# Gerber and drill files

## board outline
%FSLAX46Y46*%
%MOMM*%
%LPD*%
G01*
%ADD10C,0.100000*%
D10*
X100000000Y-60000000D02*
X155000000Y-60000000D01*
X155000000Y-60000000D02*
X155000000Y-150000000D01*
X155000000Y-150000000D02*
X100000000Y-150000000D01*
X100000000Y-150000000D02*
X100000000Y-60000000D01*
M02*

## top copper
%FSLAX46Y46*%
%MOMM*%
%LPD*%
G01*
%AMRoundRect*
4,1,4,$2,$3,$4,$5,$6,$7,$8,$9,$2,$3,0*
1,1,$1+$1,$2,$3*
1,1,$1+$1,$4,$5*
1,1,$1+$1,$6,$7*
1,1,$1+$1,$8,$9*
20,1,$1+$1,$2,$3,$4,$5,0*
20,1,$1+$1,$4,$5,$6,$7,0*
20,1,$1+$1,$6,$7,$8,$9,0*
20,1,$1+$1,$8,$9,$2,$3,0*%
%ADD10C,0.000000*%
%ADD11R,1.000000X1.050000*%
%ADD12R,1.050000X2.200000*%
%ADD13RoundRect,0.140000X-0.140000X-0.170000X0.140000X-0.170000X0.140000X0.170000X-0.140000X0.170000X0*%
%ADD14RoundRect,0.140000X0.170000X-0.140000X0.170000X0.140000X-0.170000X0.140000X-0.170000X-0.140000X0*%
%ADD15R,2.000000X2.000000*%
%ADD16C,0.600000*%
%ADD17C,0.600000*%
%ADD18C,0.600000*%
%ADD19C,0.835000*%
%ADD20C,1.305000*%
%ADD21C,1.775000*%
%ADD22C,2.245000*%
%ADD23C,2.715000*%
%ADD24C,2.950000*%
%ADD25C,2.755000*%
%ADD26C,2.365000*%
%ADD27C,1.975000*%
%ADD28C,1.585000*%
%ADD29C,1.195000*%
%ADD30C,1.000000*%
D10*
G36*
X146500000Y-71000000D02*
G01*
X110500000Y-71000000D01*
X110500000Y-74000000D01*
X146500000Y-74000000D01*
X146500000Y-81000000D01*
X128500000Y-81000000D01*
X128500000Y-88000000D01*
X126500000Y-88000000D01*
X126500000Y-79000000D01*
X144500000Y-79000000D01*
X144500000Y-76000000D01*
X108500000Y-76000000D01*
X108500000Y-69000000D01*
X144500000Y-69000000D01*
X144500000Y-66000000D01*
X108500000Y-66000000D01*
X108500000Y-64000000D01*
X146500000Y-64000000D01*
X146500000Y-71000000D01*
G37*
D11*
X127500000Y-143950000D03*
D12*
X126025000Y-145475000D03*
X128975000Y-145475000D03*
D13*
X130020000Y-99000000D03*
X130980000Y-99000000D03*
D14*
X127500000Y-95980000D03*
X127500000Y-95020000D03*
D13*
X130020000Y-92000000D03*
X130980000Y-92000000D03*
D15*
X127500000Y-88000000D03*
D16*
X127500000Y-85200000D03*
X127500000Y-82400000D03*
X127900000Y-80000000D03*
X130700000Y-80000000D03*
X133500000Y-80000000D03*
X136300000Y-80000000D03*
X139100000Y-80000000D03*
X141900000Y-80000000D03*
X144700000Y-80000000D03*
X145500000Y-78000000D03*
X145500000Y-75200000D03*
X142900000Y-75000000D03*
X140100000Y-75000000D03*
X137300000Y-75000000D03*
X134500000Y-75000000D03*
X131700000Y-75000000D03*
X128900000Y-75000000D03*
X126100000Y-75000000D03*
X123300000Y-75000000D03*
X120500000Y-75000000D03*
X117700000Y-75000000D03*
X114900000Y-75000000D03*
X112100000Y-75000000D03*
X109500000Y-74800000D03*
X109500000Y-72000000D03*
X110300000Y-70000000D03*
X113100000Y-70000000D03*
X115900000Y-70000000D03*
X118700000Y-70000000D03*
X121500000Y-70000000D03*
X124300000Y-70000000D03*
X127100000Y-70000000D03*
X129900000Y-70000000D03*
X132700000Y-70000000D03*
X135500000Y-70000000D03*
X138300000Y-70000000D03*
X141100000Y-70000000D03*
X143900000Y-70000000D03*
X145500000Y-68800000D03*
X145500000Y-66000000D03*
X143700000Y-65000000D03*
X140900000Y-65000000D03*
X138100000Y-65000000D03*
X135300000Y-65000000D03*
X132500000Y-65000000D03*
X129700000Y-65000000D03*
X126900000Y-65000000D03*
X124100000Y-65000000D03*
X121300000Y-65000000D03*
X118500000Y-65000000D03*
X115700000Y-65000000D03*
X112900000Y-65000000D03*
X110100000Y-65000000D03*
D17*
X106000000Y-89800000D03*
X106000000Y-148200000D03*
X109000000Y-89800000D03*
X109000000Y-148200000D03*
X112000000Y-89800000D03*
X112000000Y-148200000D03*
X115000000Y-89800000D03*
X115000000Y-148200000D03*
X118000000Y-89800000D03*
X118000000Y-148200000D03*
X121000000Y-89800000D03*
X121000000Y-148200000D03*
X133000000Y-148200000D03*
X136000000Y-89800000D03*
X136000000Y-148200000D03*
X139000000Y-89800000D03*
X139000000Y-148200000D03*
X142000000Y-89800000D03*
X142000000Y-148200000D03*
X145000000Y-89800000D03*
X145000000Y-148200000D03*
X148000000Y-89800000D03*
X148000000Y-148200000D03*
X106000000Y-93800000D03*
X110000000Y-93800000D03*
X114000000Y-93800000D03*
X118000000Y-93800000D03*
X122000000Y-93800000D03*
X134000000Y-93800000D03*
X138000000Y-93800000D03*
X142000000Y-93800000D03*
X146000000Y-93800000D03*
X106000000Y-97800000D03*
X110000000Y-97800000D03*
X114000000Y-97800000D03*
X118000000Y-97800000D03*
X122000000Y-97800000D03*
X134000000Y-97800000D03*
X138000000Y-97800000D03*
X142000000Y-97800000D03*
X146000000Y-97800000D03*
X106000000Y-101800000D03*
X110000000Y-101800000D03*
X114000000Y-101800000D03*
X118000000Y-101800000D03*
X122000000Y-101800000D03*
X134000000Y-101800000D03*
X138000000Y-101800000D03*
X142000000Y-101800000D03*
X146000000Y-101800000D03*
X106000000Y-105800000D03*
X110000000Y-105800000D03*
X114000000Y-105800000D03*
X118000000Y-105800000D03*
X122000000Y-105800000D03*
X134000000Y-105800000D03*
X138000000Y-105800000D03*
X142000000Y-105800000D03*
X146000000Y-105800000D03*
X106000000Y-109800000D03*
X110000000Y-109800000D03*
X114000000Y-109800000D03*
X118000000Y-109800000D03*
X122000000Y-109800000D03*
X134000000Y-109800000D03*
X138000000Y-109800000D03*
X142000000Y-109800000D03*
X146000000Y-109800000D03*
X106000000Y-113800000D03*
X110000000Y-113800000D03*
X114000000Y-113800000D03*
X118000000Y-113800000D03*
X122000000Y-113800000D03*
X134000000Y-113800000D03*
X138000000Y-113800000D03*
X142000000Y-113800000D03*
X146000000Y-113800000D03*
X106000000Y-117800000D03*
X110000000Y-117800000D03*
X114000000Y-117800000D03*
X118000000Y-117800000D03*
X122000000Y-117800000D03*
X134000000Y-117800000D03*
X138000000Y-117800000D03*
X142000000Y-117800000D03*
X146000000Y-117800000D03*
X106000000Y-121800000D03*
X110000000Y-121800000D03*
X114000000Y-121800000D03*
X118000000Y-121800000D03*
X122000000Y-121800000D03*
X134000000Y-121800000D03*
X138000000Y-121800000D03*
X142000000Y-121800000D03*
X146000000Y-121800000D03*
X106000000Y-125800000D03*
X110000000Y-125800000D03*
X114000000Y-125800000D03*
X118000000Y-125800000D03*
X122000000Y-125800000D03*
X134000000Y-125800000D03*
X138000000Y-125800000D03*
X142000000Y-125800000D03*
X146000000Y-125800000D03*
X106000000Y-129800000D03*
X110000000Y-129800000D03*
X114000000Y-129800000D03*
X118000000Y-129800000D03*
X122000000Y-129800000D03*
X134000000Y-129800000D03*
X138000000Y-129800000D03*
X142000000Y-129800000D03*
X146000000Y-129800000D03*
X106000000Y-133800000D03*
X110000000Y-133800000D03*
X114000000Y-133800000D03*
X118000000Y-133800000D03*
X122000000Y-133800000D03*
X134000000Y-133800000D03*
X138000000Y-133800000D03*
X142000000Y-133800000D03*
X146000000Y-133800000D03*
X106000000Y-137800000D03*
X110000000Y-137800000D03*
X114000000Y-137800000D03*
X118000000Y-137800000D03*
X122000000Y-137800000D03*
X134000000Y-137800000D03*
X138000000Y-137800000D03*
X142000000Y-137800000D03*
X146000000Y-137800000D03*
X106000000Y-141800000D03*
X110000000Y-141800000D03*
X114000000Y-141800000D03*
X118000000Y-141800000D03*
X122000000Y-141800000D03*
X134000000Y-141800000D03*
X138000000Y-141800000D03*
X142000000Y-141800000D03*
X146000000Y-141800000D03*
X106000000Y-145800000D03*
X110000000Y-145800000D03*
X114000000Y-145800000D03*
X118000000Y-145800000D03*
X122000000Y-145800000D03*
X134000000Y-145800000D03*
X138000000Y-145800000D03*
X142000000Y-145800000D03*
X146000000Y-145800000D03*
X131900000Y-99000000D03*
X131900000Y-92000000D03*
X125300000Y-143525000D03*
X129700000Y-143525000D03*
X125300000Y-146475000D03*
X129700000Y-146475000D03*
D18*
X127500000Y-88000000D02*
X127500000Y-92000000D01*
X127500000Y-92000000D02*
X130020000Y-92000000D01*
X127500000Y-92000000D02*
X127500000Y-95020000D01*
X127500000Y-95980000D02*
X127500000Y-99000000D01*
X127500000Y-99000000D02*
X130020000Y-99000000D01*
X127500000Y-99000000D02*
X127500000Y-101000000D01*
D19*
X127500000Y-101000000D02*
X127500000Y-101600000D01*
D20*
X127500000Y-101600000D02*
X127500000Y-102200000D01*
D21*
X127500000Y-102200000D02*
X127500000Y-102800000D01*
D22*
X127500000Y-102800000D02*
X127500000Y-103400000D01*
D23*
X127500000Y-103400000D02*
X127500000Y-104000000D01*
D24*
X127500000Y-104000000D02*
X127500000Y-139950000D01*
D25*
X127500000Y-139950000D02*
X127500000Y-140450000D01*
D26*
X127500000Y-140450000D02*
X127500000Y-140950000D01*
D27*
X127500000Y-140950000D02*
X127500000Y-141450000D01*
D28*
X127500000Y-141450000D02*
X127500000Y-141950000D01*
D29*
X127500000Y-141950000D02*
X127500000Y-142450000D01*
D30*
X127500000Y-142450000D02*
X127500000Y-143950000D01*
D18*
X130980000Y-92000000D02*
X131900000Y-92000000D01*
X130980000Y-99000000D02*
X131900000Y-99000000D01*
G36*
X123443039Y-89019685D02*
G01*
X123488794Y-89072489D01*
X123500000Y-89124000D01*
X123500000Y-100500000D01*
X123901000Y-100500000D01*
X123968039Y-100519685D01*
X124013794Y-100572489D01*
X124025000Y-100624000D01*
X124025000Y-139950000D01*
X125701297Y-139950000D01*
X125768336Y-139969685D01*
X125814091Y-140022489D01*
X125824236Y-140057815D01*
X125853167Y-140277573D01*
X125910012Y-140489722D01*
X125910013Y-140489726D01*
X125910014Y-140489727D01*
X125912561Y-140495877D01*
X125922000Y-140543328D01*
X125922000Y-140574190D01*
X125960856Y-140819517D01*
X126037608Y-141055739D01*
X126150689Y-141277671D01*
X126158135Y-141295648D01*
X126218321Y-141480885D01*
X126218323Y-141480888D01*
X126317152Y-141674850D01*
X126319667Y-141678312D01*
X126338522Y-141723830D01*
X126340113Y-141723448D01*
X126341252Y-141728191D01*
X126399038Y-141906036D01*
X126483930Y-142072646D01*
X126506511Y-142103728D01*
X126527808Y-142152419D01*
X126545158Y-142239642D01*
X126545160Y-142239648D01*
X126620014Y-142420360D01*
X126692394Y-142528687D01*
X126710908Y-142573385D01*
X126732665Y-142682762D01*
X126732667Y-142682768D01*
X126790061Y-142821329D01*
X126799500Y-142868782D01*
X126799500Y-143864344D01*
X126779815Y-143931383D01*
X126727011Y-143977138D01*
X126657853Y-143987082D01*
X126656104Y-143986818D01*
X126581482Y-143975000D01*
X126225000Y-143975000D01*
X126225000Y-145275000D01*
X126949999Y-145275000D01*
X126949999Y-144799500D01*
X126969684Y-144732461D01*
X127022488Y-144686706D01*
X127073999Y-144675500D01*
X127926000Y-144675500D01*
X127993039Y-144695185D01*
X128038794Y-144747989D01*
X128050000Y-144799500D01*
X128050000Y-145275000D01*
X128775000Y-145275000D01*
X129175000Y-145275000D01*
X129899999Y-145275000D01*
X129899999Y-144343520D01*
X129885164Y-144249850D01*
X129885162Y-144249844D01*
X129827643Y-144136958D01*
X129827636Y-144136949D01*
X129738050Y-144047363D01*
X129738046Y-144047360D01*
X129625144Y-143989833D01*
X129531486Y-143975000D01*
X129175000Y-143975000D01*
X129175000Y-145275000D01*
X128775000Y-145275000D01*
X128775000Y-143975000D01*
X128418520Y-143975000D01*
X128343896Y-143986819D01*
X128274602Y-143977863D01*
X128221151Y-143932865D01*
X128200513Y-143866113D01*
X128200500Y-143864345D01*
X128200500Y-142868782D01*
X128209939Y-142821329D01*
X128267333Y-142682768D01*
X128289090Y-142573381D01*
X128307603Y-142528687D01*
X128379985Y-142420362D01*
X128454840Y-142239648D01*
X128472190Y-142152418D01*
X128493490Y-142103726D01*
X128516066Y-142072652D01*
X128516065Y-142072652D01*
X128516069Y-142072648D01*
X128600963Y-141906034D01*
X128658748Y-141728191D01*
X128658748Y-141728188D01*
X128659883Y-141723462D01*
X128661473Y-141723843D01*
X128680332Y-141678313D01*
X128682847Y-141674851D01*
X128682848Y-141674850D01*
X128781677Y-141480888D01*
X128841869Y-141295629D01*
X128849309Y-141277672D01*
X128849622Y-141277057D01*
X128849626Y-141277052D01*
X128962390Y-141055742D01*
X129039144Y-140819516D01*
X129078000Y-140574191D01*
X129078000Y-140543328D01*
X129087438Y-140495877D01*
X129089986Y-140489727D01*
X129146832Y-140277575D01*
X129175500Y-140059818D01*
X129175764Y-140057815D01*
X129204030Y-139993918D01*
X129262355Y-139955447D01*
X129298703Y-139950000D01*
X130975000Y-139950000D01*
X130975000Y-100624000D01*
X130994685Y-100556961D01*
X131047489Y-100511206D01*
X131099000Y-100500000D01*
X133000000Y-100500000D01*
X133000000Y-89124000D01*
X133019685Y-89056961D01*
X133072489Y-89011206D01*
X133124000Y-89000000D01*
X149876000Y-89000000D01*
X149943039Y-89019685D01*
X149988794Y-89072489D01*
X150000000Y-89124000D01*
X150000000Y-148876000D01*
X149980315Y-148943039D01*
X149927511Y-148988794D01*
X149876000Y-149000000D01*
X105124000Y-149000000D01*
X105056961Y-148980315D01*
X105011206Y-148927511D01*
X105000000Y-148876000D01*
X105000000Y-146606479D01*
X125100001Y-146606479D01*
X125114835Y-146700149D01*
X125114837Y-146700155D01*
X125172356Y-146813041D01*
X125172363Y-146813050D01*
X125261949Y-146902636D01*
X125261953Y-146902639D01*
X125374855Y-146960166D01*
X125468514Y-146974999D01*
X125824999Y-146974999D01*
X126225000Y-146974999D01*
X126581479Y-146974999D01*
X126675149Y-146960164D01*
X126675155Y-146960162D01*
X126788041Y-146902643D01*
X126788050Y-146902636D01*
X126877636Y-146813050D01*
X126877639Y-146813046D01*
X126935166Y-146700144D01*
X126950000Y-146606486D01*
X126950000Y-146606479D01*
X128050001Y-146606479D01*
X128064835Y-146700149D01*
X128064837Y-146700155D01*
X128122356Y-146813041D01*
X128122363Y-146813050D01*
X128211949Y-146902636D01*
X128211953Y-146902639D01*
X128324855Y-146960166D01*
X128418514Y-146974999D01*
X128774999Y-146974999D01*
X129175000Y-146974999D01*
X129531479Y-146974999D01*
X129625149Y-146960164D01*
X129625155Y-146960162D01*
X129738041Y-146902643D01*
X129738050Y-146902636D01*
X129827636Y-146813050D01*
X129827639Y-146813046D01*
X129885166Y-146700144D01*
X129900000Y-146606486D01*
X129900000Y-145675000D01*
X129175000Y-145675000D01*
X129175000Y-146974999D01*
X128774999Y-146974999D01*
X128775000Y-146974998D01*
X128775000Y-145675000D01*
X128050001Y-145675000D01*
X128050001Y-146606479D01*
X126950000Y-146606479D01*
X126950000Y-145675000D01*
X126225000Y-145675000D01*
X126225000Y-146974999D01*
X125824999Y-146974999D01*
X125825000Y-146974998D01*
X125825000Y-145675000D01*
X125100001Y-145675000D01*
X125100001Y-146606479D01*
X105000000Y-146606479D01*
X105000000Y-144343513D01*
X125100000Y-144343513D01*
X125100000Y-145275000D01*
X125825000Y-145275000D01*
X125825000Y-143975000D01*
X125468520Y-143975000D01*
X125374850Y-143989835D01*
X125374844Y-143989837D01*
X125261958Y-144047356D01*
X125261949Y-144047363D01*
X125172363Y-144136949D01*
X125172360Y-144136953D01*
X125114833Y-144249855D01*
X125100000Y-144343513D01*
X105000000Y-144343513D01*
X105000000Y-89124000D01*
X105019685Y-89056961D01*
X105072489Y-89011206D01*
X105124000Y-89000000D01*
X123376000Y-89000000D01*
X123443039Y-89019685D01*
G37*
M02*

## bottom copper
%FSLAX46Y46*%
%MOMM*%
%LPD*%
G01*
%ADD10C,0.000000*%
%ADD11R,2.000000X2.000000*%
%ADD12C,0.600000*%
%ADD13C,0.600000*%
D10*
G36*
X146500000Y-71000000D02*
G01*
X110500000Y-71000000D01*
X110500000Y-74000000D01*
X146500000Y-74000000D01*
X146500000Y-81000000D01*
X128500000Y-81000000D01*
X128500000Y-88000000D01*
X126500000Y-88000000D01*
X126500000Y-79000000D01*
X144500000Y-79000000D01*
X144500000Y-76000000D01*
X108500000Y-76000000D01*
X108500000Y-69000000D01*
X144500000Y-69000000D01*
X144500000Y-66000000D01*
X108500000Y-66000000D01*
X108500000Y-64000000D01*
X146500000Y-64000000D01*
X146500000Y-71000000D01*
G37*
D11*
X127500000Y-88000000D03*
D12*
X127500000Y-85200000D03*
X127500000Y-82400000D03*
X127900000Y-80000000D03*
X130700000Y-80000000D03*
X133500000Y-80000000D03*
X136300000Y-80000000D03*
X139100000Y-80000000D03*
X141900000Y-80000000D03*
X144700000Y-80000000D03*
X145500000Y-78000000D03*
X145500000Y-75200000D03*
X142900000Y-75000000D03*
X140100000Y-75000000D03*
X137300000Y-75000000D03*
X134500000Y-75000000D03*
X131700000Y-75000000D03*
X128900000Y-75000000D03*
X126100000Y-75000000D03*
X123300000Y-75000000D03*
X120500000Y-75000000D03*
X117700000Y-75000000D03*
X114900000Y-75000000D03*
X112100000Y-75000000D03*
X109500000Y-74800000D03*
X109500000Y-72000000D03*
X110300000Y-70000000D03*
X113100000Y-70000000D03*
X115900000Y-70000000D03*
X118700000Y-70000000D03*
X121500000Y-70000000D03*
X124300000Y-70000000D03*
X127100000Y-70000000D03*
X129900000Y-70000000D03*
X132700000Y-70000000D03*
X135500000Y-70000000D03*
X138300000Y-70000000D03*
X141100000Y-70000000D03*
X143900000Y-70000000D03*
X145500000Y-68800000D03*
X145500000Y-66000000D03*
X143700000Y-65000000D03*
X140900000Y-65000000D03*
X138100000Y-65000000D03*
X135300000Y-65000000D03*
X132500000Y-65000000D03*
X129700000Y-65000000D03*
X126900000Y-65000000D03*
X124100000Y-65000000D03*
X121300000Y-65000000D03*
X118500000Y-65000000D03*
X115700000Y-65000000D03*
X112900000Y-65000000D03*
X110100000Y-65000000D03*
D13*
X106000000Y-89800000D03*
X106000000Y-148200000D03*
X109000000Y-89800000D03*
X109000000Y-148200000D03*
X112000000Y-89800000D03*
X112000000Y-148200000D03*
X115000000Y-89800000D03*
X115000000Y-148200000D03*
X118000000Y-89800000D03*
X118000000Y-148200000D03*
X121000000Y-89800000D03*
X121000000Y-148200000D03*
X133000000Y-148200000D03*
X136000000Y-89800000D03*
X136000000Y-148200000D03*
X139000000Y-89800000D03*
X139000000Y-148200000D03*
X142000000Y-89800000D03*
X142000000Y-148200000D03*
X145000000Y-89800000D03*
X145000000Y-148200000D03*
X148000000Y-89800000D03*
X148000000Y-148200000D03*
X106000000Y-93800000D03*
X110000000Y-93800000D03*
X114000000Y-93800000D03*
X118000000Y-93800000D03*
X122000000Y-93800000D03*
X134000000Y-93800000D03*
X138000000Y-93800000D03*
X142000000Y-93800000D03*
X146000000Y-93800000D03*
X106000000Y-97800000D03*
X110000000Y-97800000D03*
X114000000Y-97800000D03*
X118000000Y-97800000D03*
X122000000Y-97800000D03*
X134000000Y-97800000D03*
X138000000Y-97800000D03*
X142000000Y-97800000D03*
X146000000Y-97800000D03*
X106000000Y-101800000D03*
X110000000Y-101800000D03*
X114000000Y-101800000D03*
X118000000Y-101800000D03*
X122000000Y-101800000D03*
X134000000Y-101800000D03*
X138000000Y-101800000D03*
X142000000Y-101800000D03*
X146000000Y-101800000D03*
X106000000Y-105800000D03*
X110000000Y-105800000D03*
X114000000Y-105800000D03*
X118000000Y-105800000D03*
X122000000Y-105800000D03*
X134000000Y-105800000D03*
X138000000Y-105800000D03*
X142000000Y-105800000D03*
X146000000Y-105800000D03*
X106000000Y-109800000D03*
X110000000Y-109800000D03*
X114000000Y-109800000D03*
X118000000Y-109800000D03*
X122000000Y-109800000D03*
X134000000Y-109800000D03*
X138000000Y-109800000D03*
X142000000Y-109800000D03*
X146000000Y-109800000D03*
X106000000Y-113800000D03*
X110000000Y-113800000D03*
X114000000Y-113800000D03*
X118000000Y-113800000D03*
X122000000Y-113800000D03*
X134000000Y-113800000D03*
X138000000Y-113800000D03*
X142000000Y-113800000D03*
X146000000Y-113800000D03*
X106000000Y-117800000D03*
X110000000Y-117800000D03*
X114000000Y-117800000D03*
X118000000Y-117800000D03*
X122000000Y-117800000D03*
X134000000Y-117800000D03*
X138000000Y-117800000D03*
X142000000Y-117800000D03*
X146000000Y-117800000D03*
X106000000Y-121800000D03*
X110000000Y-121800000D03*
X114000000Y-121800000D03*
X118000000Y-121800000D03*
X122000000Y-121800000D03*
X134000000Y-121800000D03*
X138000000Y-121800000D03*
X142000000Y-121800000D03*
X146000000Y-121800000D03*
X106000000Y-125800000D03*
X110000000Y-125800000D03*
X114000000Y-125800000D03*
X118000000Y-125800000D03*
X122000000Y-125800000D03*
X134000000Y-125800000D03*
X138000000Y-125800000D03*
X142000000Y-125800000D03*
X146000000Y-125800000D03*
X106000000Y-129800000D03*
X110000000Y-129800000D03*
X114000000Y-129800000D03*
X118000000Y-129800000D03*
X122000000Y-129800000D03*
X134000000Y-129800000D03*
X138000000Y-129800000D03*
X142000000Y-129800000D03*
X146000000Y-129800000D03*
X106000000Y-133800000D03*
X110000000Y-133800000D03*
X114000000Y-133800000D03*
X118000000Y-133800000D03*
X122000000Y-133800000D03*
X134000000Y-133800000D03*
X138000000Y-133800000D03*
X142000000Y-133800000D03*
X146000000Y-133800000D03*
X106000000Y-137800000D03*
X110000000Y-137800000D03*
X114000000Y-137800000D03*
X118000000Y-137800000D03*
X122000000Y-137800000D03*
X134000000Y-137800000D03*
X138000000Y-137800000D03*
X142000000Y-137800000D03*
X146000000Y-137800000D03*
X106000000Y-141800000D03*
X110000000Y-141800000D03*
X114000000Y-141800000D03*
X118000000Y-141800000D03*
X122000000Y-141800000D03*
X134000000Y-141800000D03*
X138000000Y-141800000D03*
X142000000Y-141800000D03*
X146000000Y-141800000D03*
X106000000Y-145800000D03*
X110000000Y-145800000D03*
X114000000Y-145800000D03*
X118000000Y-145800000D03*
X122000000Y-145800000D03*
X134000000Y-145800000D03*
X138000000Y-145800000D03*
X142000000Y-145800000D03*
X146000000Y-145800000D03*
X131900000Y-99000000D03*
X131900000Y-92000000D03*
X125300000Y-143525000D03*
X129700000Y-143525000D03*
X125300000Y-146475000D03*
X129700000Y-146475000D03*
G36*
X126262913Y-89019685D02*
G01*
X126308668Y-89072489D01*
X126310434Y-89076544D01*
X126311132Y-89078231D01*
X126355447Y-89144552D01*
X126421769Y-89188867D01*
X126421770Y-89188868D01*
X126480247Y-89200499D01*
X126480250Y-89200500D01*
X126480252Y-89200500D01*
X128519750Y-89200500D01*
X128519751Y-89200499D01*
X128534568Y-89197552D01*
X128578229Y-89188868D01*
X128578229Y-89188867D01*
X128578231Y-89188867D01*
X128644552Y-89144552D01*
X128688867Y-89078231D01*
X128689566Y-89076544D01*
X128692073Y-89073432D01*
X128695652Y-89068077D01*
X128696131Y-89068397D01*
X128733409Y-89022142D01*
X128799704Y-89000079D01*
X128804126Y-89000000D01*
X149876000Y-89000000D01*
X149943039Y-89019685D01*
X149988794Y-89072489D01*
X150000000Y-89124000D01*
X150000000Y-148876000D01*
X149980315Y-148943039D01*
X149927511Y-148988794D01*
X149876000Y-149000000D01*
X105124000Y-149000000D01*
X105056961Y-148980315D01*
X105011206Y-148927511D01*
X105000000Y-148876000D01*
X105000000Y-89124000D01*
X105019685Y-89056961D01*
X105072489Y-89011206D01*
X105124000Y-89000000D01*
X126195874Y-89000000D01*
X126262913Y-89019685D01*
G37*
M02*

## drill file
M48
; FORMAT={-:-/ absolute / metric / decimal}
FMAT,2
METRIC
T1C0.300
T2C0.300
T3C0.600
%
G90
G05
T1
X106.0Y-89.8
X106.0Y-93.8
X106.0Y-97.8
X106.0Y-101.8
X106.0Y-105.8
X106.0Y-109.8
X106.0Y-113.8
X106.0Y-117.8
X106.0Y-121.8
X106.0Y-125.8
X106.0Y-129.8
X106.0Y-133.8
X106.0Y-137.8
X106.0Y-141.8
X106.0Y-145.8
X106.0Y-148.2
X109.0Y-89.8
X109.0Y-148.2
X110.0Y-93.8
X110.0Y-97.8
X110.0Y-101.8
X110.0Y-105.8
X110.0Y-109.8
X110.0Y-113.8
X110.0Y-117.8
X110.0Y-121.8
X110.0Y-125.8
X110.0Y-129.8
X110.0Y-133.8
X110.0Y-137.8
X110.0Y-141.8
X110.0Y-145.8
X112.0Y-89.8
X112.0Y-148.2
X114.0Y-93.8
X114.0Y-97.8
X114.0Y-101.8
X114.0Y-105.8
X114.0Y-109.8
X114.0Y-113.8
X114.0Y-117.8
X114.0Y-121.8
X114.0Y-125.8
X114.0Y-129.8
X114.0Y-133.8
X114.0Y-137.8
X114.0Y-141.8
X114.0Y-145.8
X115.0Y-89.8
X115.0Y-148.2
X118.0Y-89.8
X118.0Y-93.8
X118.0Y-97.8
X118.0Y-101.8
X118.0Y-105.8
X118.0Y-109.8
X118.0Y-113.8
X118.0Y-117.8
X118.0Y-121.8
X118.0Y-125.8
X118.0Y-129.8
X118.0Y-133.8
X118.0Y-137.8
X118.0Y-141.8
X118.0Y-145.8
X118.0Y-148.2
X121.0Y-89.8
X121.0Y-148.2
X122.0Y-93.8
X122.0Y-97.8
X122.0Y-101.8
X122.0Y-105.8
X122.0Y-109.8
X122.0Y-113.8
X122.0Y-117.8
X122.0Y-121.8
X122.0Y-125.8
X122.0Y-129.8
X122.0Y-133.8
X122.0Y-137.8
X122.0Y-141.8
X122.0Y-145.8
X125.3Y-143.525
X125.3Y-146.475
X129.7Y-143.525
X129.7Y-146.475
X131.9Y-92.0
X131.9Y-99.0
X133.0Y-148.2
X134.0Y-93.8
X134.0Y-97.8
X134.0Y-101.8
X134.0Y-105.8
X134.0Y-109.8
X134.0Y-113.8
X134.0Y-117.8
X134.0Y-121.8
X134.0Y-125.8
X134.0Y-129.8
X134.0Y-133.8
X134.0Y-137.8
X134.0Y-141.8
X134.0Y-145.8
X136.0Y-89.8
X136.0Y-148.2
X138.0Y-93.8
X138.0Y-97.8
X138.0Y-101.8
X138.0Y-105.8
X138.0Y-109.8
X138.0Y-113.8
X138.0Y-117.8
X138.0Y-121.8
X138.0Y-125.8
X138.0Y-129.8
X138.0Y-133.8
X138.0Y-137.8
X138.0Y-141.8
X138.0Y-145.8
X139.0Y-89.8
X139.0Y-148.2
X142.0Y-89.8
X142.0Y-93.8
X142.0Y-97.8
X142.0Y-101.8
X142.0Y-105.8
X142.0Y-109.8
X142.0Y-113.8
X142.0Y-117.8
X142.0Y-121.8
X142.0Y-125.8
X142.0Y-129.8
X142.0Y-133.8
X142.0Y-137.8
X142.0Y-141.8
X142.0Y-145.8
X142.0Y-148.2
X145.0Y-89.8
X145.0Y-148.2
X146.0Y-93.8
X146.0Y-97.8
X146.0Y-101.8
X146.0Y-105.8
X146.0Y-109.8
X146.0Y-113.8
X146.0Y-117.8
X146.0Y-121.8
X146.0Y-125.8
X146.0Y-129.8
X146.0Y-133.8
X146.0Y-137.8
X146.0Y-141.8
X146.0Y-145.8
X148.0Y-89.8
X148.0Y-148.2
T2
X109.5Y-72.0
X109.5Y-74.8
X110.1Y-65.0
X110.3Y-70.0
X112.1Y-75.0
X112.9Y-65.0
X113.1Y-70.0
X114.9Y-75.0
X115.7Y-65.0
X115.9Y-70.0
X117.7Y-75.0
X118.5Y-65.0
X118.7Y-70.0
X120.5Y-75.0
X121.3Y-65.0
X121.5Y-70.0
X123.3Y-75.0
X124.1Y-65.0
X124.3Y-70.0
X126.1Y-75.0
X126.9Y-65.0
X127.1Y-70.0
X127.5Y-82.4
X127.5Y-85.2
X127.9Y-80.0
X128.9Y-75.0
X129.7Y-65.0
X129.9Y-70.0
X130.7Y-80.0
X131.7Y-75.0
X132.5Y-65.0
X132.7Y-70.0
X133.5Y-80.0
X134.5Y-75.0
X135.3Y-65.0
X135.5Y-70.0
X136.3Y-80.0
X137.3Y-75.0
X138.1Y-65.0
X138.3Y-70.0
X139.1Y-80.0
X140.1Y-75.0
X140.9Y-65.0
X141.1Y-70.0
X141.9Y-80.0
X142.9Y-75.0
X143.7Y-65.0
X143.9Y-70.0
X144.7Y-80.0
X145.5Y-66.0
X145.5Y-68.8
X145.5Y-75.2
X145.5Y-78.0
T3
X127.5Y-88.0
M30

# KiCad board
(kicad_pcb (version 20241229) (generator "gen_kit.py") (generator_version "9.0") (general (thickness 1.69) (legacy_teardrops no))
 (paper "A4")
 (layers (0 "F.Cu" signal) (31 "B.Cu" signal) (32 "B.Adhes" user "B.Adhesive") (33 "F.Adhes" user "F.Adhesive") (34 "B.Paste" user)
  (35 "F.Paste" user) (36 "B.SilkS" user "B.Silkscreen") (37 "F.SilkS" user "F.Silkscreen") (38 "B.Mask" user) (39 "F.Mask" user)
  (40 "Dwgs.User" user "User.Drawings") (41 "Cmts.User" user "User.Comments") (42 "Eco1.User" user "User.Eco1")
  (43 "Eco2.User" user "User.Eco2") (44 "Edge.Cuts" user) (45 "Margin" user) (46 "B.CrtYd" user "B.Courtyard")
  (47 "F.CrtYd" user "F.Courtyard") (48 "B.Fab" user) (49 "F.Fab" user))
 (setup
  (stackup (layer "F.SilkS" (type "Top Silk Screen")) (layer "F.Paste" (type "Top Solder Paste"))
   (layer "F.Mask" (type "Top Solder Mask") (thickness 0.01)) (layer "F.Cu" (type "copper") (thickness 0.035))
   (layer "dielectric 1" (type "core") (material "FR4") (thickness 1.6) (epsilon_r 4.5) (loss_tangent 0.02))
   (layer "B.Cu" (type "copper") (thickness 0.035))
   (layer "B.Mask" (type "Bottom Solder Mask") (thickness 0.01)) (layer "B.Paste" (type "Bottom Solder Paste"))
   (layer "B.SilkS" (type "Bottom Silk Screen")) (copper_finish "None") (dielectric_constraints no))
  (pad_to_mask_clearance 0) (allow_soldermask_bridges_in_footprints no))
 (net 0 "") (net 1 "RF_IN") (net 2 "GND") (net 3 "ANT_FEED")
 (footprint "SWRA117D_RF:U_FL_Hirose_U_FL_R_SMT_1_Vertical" (layer "F.Cu") (at 127.5 145 270)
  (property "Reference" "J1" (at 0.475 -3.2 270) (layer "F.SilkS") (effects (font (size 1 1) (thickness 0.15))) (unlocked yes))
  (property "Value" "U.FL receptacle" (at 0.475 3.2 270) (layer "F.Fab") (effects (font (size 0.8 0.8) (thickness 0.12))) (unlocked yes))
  (pad "1" smd rect (at -1.05 0 270) (size 1.05 1) (layers "F.Cu" "F.Paste" "F.Mask") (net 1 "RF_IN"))
  (pad "2" smd rect (at 0.475 1.475 270) (size 2.2 1.05) (layers "F.Cu" "F.Paste" "F.Mask") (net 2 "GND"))
  (pad "2" smd rect (at 0.475 -1.475 270) (size 2.2 1.05) (layers "F.Cu" "F.Paste" "F.Mask") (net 2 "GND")))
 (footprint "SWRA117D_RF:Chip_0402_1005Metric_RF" (layer "F.Cu") (at 130.5 99)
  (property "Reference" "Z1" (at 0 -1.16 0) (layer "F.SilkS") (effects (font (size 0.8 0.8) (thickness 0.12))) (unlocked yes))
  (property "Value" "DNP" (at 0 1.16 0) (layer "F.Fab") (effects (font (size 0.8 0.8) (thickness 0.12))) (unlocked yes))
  (pad "1" smd roundrect (at -0.48 0) (size 0.56 0.62) (layers "F.Cu" "F.Paste" "F.Mask") (roundrect_rratio 0.25) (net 1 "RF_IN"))
  (pad "2" smd roundrect (at 0.48 0) (size 0.56 0.62) (layers "F.Cu" "F.Paste" "F.Mask") (roundrect_rratio 0.25) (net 2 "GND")))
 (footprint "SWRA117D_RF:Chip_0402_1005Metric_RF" (layer "F.Cu") (at 127.5 95.5 90)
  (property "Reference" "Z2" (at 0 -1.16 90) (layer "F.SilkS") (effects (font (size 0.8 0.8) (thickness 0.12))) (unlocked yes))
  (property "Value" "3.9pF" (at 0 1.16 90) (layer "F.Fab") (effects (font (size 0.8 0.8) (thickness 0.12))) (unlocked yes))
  (pad "1" smd roundrect (at -0.48 0 90) (size 0.56 0.62) (layers "F.Cu" "F.Paste" "F.Mask") (roundrect_rratio 0.25) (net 1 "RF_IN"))
  (pad "2" smd roundrect (at 0.48 0 90) (size 0.56 0.62) (layers "F.Cu" "F.Paste" "F.Mask") (roundrect_rratio 0.25) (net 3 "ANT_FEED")))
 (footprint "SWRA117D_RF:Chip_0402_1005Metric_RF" (layer "F.Cu") (at 130.5 92)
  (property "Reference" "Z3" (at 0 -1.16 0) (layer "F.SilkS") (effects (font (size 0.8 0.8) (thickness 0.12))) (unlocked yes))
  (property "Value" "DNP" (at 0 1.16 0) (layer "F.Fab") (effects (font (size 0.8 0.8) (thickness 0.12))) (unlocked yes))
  (pad "1" smd roundrect (at -0.48 0) (size 0.56 0.62) (layers "F.Cu" "F.Paste" "F.Mask") (roundrect_rratio 0.25) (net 3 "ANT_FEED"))
  (pad "2" smd roundrect (at 0.48 0) (size 0.56 0.62) (layers "F.Cu" "F.Paste" "F.Mask") (roundrect_rratio 0.25) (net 2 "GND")))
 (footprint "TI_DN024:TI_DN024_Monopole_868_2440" (layer "F.Cu") (at 127.5 88)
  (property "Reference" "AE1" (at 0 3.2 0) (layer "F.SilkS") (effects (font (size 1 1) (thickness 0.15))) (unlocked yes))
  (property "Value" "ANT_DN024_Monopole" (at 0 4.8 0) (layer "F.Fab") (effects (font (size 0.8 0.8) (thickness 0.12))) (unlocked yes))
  (fp_poly
   (pts (xy 1 0) (xy 1 -7) (xy 19 -7) (xy 19 -14) (xy -17 -14) (xy -17 -17) (xy 19 -17) (xy 19 -24) (xy -19 -24) (xy -19 -22) (xy 17 -22)
    (xy 17 -19) (xy -19 -19) (xy -19 -12) (xy 17 -12) (xy 17 -9) (xy -1 -9) (xy -1 0))
   (stroke (width 0) (type solid)) (fill yes) (layer "F.Cu"))
  (fp_poly
   (pts (xy 1 0) (xy 1 -7) (xy 19 -7) (xy 19 -14) (xy -17 -14) (xy -17 -17) (xy 19 -17) (xy 19 -24) (xy -19 -24) (xy -19 -22) (xy 17 -22)
    (xy 17 -19) (xy -19 -19) (xy -19 -12) (xy 17 -12) (xy 17 -9) (xy -1 -9) (xy -1 0))
   (stroke (width 0) (type solid)) (fill yes) (layer "B.Cu"))
  (pad "1" thru_hole rect (at 0 0) (size 2 2) (drill 0.6) (layers "*.Cu" "*.Mask") (remove_unused_layers no) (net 3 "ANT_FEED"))
  (pad "1" thru_hole circle (at 0 -2.8) (size 0.6 0.6) (drill 0.3) (layers "*.Cu") (remove_unused_layers no) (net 3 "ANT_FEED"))
  (pad "1" thru_hole circle (at 0 -5.6) (size 0.6 0.6) (drill 0.3) (layers "*.Cu") (remove_unused_layers no) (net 3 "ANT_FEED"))
  (pad "1" thru_hole circle (at 0.4 -8) (size 0.6 0.6) (drill 0.3) (layers "*.Cu") (remove_unused_layers no) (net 3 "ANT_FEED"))
  (pad "1" thru_hole circle (at 3.2 -8) (size 0.6 0.6) (drill 0.3) (layers "*.Cu") (remove_unused_layers no) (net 3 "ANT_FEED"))
  (pad "1" thru_hole circle (at 6 -8) (size 0.6 0.6) (drill 0.3) (layers "*.Cu") (remove_unused_layers no) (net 3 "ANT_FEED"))
  (pad "1" thru_hole circle (at 8.8 -8) (size 0.6 0.6) (drill 0.3) (layers "*.Cu") (remove_unused_layers no) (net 3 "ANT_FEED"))
  (pad "1" thru_hole circle (at 11.6 -8) (size 0.6 0.6) (drill 0.3) (layers "*.Cu") (remove_unused_layers no) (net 3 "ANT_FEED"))
  (pad "1" thru_hole circle (at 14.4 -8) (size 0.6 0.6) (drill 0.3) (layers "*.Cu") (remove_unused_layers no) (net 3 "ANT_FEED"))
  (pad "1" thru_hole circle (at 17.2 -8) (size 0.6 0.6) (drill 0.3) (layers "*.Cu") (remove_unused_layers no) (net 3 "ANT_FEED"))
  (pad "1" thru_hole circle (at 18 -10) (size 0.6 0.6) (drill 0.3) (layers "*.Cu") (remove_unused_layers no) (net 3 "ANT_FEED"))
  (pad "1" thru_hole circle (at 18 -12.8) (size 0.6 0.6) (drill 0.3) (layers "*.Cu") (remove_unused_layers no) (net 3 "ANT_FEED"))
  (pad "1" thru_hole circle (at 15.4 -13) (size 0.6 0.6) (drill 0.3) (layers "*.Cu") (remove_unused_layers no) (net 3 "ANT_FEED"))
  (pad "1" thru_hole circle (at 12.6 -13) (size 0.6 0.6) (drill 0.3) (layers "*.Cu") (remove_unused_layers no) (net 3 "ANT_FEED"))
  (pad "1" thru_hole circle (at 9.8 -13) (size 0.6 0.6) (drill 0.3) (layers "*.Cu") (remove_unused_layers no) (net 3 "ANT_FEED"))
  (pad "1" thru_hole circle (at 7 -13) (size 0.6 0.6) (drill 0.3) (layers "*.Cu") (remove_unused_layers no) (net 3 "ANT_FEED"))
  (pad "1" thru_hole circle (at 4.2 -13) (size 0.6 0.6) (drill 0.3) (layers "*.Cu") (remove_unused_layers no) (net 3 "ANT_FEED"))
  (pad "1" thru_hole circle (at 1.4 -13) (size 0.6 0.6) (drill 0.3) (layers "*.Cu") (remove_unused_layers no) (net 3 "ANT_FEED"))
  (pad "1" thru_hole circle (at -1.4 -13) (size 0.6 0.6) (drill 0.3) (layers "*.Cu") (remove_unused_layers no) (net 3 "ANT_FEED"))
  (pad "1" thru_hole circle (at -4.2 -13) (size 0.6 0.6) (drill 0.3) (layers "*.Cu") (remove_unused_layers no) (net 3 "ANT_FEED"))
  (pad "1" thru_hole circle (at -7 -13) (size 0.6 0.6) (drill 0.3) (layers "*.Cu") (remove_unused_layers no) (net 3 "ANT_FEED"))
  (pad "1" thru_hole circle (at -9.8 -13) (size 0.6 0.6) (drill 0.3) (layers "*.Cu") (remove_unused_layers no) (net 3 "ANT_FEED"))
  (pad "1" thru_hole circle (at -12.6 -13) (size 0.6 0.6) (drill 0.3) (layers "*.Cu") (remove_unused_layers no) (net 3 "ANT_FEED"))
  (pad "1" thru_hole circle (at -15.4 -13) (size 0.6 0.6) (drill 0.3) (layers "*.Cu") (remove_unused_layers no) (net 3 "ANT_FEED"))
  (pad "1" thru_hole circle (at -18 -13.2) (size 0.6 0.6) (drill 0.3) (layers "*.Cu") (remove_unused_layers no) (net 3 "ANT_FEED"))
  (pad "1" thru_hole circle (at -18 -16) (size 0.6 0.6) (drill 0.3) (layers "*.Cu") (remove_unused_layers no) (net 3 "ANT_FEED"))
  (pad "1" thru_hole circle (at -17.2 -18) (size 0.6 0.6) (drill 0.3) (layers "*.Cu") (remove_unused_layers no) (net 3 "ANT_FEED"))
  (pad "1" thru_hole circle (at -14.4 -18) (size 0.6 0.6) (drill 0.3) (layers "*.Cu") (remove_unused_layers no) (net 3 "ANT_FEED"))
  (pad "1" thru_hole circle (at -11.6 -18) (size 0.6 0.6) (drill 0.3) (layers "*.Cu") (remove_unused_layers no) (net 3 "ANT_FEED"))
  (pad "1" thru_hole circle (at -8.8 -18) (size 0.6 0.6) (drill 0.3) (layers "*.Cu") (remove_unused_layers no) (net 3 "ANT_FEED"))
  (pad "1" thru_hole circle (at -6 -18) (size 0.6 0.6) (drill 0.3) (layers "*.Cu") (remove_unused_layers no) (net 3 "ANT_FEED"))
  (pad "1" thru_hole circle (at -3.2 -18) (size 0.6 0.6) (drill 0.3) (layers "*.Cu") (remove_unused_layers no) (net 3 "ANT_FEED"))
  (pad "1" thru_hole circle (at -0.4 -18) (size 0.6 0.6) (drill 0.3) (layers "*.Cu") (remove_unused_layers no) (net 3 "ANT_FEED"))
  (pad "1" thru_hole circle (at 2.4 -18) (size 0.6 0.6) (drill 0.3) (layers "*.Cu") (remove_unused_layers no) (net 3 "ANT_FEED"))
  (pad "1" thru_hole circle (at 5.2 -18) (size 0.6 0.6) (drill 0.3) (layers "*.Cu") (remove_unused_layers no) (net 3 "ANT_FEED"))
  (pad "1" thru_hole circle (at 8 -18) (size 0.6 0.6) (drill 0.3) (layers "*.Cu") (remove_unused_layers no) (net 3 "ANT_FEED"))
  (pad "1" thru_hole circle (at 10.8 -18) (size 0.6 0.6) (drill 0.3) (layers "*.Cu") (remove_unused_layers no) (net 3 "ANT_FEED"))
  (pad "1" thru_hole circle (at 13.6 -18) (size 0.6 0.6) (drill 0.3) (layers "*.Cu") (remove_unused_layers no) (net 3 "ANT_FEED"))
  (pad "1" thru_hole circle (at 16.4 -18) (size 0.6 0.6) (drill 0.3) (layers "*.Cu") (remove_unused_layers no) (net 3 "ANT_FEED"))
  (pad "1" thru_hole circle (at 18 -19.2) (size 0.6 0.6) (drill 0.3) (layers "*.Cu") (remove_unused_layers no) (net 3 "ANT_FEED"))
  (pad "1" thru_hole circle (at 18 -22) (size 0.6 0.6) (drill 0.3) (layers "*.Cu") (remove_unused_layers no) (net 3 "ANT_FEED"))
  (pad "1" thru_hole circle (at 16.2 -23) (size 0.6 0.6) (drill 0.3) (layers "*.Cu") (remove_unused_layers no) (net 3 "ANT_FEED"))
  (pad "1" thru_hole circle (at 13.4 -23) (size 0.6 0.6) (drill 0.3) (layers "*.Cu") (remove_unused_layers no) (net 3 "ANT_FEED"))
  (pad "1" thru_hole circle (at 10.6 -23) (size 0.6 0.6) (drill 0.3) (layers "*.Cu") (remove_unused_layers no) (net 3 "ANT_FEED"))
  (pad "1" thru_hole circle (at 7.8 -23) (size 0.6 0.6) (drill 0.3) (layers "*.Cu") (remove_unused_layers no) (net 3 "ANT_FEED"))
  (pad "1" thru_hole circle (at 5 -23) (size 0.6 0.6) (drill 0.3) (layers "*.Cu") (remove_unused_layers no) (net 3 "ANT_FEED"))
  (pad "1" thru_hole circle (at 2.2 -23) (size 0.6 0.6) (drill 0.3) (layers "*.Cu") (remove_unused_layers no) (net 3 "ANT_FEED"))
  (pad "1" thru_hole circle (at -0.6 -23) (size 0.6 0.6) (drill 0.3) (layers "*.Cu") (remove_unused_layers no) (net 3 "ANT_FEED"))
  (pad "1" thru_hole circle (at -3.4 -23) (size 0.6 0.6) (drill 0.3) (layers "*.Cu") (remove_unused_layers no) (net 3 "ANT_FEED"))
  (pad "1" thru_hole circle (at -6.2 -23) (size 0.6 0.6) (drill 0.3) (layers "*.Cu") (remove_unused_layers no) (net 3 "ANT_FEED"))
  (pad "1" thru_hole circle (at -9 -23) (size 0.6 0.6) (drill 0.3) (layers "*.Cu") (remove_unused_layers no) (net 3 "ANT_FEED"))
  (pad "1" thru_hole circle (at -11.8 -23) (size 0.6 0.6) (drill 0.3) (layers "*.Cu") (remove_unused_layers no) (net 3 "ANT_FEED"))
  (pad "1" thru_hole circle (at -14.6 -23) (size 0.6 0.6) (drill 0.3) (layers "*.Cu") (remove_unused_layers no) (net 3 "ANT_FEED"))
  (pad "1" thru_hole circle (at -17.4 -23) (size 0.6 0.6) (drill 0.3) (layers "*.Cu") (remove_unused_layers no) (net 3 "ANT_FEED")))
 (gr_line (start 100 60) (end 155 60) (stroke (width 0.1) (type solid)) (layer "Edge.Cuts"))
 (gr_line (start 155 60) (end 155 150) (stroke (width 0.1) (type solid)) (layer "Edge.Cuts"))
 (gr_line (start 155 150) (end 100 150) (stroke (width 0.1) (type solid)) (layer "Edge.Cuts"))
 (gr_line (start 100 150) (end 100 60) (stroke (width 0.1) (type solid)) (layer "Edge.Cuts"))
 (segment (start 127.5 88) (end 127.5 92) (width 0.6) (layer "F.Cu") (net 3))
 (segment (start 127.5 92) (end 130.02 92) (width 0.6) (layer "F.Cu") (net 3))
 (segment (start 127.5 92) (end 127.5 95.02) (width 0.6) (layer "F.Cu") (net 3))
 (segment (start 127.5 95.98) (end 127.5 99) (width 0.6) (layer "F.Cu") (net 1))
 (segment (start 127.5 99) (end 130.02 99) (width 0.6) (layer "F.Cu") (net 1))
 (segment (start 127.5 99) (end 127.5 101) (width 0.6) (layer "F.Cu") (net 1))
 (segment (start 127.5 101) (end 127.5 101.6) (width 0.835) (layer "F.Cu") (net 1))
 (segment (start 127.5 101.6) (end 127.5 102.2) (width 1.305) (layer "F.Cu") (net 1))
 (segment (start 127.5 102.2) (end 127.5 102.8) (width 1.775) (layer "F.Cu") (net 1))
 (segment (start 127.5 102.8) (end 127.5 103.4) (width 2.245) (layer "F.Cu") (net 1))
 (segment (start 127.5 103.4) (end 127.5 104) (width 2.715) (layer "F.Cu") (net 1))
 (segment (start 127.5 104) (end 127.5 139.95) (width 2.95) (layer "F.Cu") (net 1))
 (segment (start 127.5 139.95) (end 127.5 140.45) (width 2.755) (layer "F.Cu") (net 1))
 (segment (start 127.5 140.45) (end 127.5 140.95) (width 2.365) (layer "F.Cu") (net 1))
 (segment (start 127.5 140.95) (end 127.5 141.45) (width 1.975) (layer "F.Cu") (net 1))
 (segment (start 127.5 141.45) (end 127.5 141.95) (width 1.585) (layer "F.Cu") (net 1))
 (segment (start 127.5 141.95) (end 127.5 142.45) (width 1.195) (layer "F.Cu") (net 1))
 (segment (start 127.5 142.45) (end 127.5 143.95) (width 1) (layer "F.Cu") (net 1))
 (segment (start 130.98 92) (end 131.9 92) (width 0.6) (layer "F.Cu") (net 2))
 (segment (start 130.98 99) (end 131.9 99) (width 0.6) (layer "F.Cu") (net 2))
 (via (at 106 89.8) (size 0.6) (drill 0.3) (layers "F.Cu" "B.Cu") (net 2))
 (via (at 106 148.2) (size 0.6) (drill 0.3) (layers "F.Cu" "B.Cu") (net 2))
 (via (at 109 89.8) (size 0.6) (drill 0.3) (layers "F.Cu" "B.Cu") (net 2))
 (via (at 109 148.2) (size 0.6) (drill 0.3) (layers "F.Cu" "B.Cu") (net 2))
 (via (at 112 89.8) (size 0.6) (drill 0.3) (layers "F.Cu" "B.Cu") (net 2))
 (via (at 112 148.2) (size 0.6) (drill 0.3) (layers "F.Cu" "B.Cu") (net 2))
 (via (at 115 89.8) (size 0.6) (drill 0.3) (layers "F.Cu" "B.Cu") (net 2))
 (via (at 115 148.2) (size 0.6) (drill 0.3) (layers "F.Cu" "B.Cu") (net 2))
 (via (at 118 89.8) (size 0.6) (drill 0.3) (layers "F.Cu" "B.Cu") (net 2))
 (via (at 118 148.2) (size 0.6) (drill 0.3) (layers "F.Cu" "B.Cu") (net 2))
 (via (at 121 89.8) (size 0.6) (drill 0.3) (layers "F.Cu" "B.Cu") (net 2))
 (via (at 121 148.2) (size 0.6) (drill 0.3) (layers "F.Cu" "B.Cu") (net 2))
 (via (at 133 148.2) (size 0.6) (drill 0.3) (layers "F.Cu" "B.Cu") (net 2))
 (via (at 136 89.8) (size 0.6) (drill 0.3) (layers "F.Cu" "B.Cu") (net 2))
 (via (at 136 148.2) (size 0.6) (drill 0.3) (layers "F.Cu" "B.Cu") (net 2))
 (via (at 139 89.8) (size 0.6) (drill 0.3) (layers "F.Cu" "B.Cu") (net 2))
 (via (at 139 148.2) (size 0.6) (drill 0.3) (layers "F.Cu" "B.Cu") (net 2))
 (via (at 142 89.8) (size 0.6) (drill 0.3) (layers "F.Cu" "B.Cu") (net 2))
 (via (at 142 148.2) (size 0.6) (drill 0.3) (layers "F.Cu" "B.Cu") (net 2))
 (via (at 145 89.8) (size 0.6) (drill 0.3) (layers "F.Cu" "B.Cu") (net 2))
 (via (at 145 148.2) (size 0.6) (drill 0.3) (layers "F.Cu" "B.Cu") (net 2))
 (via (at 148 89.8) (size 0.6) (drill 0.3) (layers "F.Cu" "B.Cu") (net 2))
 (via (at 148 148.2) (size 0.6) (drill 0.3) (layers "F.Cu" "B.Cu") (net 2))
 (via (at 106 93.8) (size 0.6) (drill 0.3) (layers "F.Cu" "B.Cu") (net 2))
 (via (at 110 93.8) (size 0.6) (drill 0.3) (layers "F.Cu" "B.Cu") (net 2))
 (via (at 114 93.8) (size 0.6) (drill 0.3) (layers "F.Cu" "B.Cu") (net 2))
 (via (at 118 93.8) (size 0.6) (drill 0.3) (layers "F.Cu" "B.Cu") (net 2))
 (via (at 122 93.8) (size 0.6) (drill 0.3) (layers "F.Cu" "B.Cu") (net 2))
 (via (at 134 93.8) (size 0.6) (drill 0.3) (layers "F.Cu" "B.Cu") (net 2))
 (via (at 138 93.8) (size 0.6) (drill 0.3) (layers "F.Cu" "B.Cu") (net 2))
 (via (at 142 93.8) (size 0.6) (drill 0.3) (layers "F.Cu" "B.Cu") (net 2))
 (via (at 146 93.8) (size 0.6) (drill 0.3) (layers "F.Cu" "B.Cu") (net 2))
 (via (at 106 97.8) (size 0.6) (drill 0.3) (layers "F.Cu" "B.Cu") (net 2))
 (via (at 110 97.8) (size 0.6) (drill 0.3) (layers "F.Cu" "B.Cu") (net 2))
 (via (at 114 97.8) (size 0.6) (drill 0.3) (layers "F.Cu" "B.Cu") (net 2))
 (via (at 118 97.8) (size 0.6) (drill 0.3) (layers "F.Cu" "B.Cu") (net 2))
 (via (at 122 97.8) (size 0.6) (drill 0.3) (layers "F.Cu" "B.Cu") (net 2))
 (via (at 134 97.8) (size 0.6) (drill 0.3) (layers "F.Cu" "B.Cu") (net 2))
 (via (at 138 97.8) (size 0.6) (drill 0.3) (layers "F.Cu" "B.Cu") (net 2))
 (via (at 142 97.8) (size 0.6) (drill 0.3) (layers "F.Cu" "B.Cu") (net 2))
 (via (at 146 97.8) (size 0.6) (drill 0.3) (layers "F.Cu" "B.Cu") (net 2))
 (via (at 106 101.8) (size 0.6) (drill 0.3) (layers "F.Cu" "B.Cu") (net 2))
 (via (at 110 101.8) (size 0.6) (drill 0.3) (layers "F.Cu" "B.Cu") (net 2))
 (via (at 114 101.8) (size 0.6) (drill 0.3) (layers "F.Cu" "B.Cu") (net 2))
 (via (at 118 101.8) (size 0.6) (drill 0.3) (layers "F.Cu" "B.Cu") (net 2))
 (via (at 122 101.8) (size 0.6) (drill 0.3) (layers "F.Cu" "B.Cu") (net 2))
 (via (at 134 101.8) (size 0.6) (drill 0.3) (layers "F.Cu" "B.Cu") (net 2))
 (via (at 138 101.8) (size 0.6) (drill 0.3) (layers "F.Cu" "B.Cu") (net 2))
 (via (at 142 101.8) (size 0.6) (drill 0.3) (layers "F.Cu" "B.Cu") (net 2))
 (via (at 146 101.8) (size 0.6) (drill 0.3) (layers "F.Cu" "B.Cu") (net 2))
 (via (at 106 105.8) (size 0.6) (drill 0.3) (layers "F.Cu" "B.Cu") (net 2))
 (via (at 110 105.8) (size 0.6) (drill 0.3) (layers "F.Cu" "B.Cu") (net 2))
 (via (at 114 105.8) (size 0.6) (drill 0.3) (layers "F.Cu" "B.Cu") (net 2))
 (via (at 118 105.8) (size 0.6) (drill 0.3) (layers "F.Cu" "B.Cu") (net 2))
 (via (at 122 105.8) (size 0.6) (drill 0.3) (layers "F.Cu" "B.Cu") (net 2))
 (via (at 134 105.8) (size 0.6) (drill 0.3) (layers "F.Cu" "B.Cu") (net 2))
 (via (at 138 105.8) (size 0.6) (drill 0.3) (layers "F.Cu" "B.Cu") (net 2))
 (via (at 142 105.8) (size 0.6) (drill 0.3) (layers "F.Cu" "B.Cu") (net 2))
 (via (at 146 105.8) (size 0.6) (drill 0.3) (layers "F.Cu" "B.Cu") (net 2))
 (via (at 106 109.8) (size 0.6) (drill 0.3) (layers "F.Cu" "B.Cu") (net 2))
 (via (at 110 109.8) (size 0.6) (drill 0.3) (layers "F.Cu" "B.Cu") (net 2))
 (via (at 114 109.8) (size 0.6) (drill 0.3) (layers "F.Cu" "B.Cu") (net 2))
 (via (at 118 109.8) (size 0.6) (drill 0.3) (layers "F.Cu" "B.Cu") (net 2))
 (via (at 122 109.8) (size 0.6) (drill 0.3) (layers "F.Cu" "B.Cu") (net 2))
 (via (at 134 109.8) (size 0.6) (drill 0.3) (layers "F.Cu" "B.Cu") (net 2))
 (via (at 138 109.8) (size 0.6) (drill 0.3) (layers "F.Cu" "B.Cu") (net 2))
 (via (at 142 109.8) (size 0.6) (drill 0.3) (layers "F.Cu" "B.Cu") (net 2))
 (via (at 146 109.8) (size 0.6) (drill 0.3) (layers "F.Cu" "B.Cu") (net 2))
 (via (at 106 113.8) (size 0.6) (drill 0.3) (layers "F.Cu" "B.Cu") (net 2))
 (via (at 110 113.8) (size 0.6) (drill 0.3) (layers "F.Cu" "B.Cu") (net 2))
 (via (at 114 113.8) (size 0.6) (drill 0.3) (layers "F.Cu" "B.Cu") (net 2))
 (via (at 118 113.8) (size 0.6) (drill 0.3) (layers "F.Cu" "B.Cu") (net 2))
 (via (at 122 113.8) (size 0.6) (drill 0.3) (layers "F.Cu" "B.Cu") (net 2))
 (via (at 134 113.8) (size 0.6) (drill 0.3) (layers "F.Cu" "B.Cu") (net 2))
 (via (at 138 113.8) (size 0.6) (drill 0.3) (layers "F.Cu" "B.Cu") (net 2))
 (via (at 142 113.8) (size 0.6) (drill 0.3) (layers "F.Cu" "B.Cu") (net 2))
 (via (at 146 113.8) (size 0.6) (drill 0.3) (layers "F.Cu" "B.Cu") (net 2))
 (via (at 106 117.8) (size 0.6) (drill 0.3) (layers "F.Cu" "B.Cu") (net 2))
 (via (at 110 117.8) (size 0.6) (drill 0.3) (layers "F.Cu" "B.Cu") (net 2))
 (via (at 114 117.8) (size 0.6) (drill 0.3) (layers "F.Cu" "B.Cu") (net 2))
 (via (at 118 117.8) (size 0.6) (drill 0.3) (layers "F.Cu" "B.Cu") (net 2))
 (via (at 122 117.8) (size 0.6) (drill 0.3) (layers "F.Cu" "B.Cu") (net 2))
 (via (at 134 117.8) (size 0.6) (drill 0.3) (layers "F.Cu" "B.Cu") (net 2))
 (via (at 138 117.8) (size 0.6) (drill 0.3) (layers "F.Cu" "B.Cu") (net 2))
 (via (at 142 117.8) (size 0.6) (drill 0.3) (layers "F.Cu" "B.Cu") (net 2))
 (via (at 146 117.8) (size 0.6) (drill 0.3) (layers "F.Cu" "B.Cu") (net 2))
 (via (at 106 121.8) (size 0.6) (drill 0.3) (layers "F.Cu" "B.Cu") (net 2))
 (via (at 110 121.8) (size 0.6) (drill 0.3) (layers "F.Cu" "B.Cu") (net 2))
 (via (at 114 121.8) (size 0.6) (drill 0.3) (layers "F.Cu" "B.Cu") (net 2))
 (via (at 118 121.8) (size 0.6) (drill 0.3) (layers "F.Cu" "B.Cu") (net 2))
 (via (at 122 121.8) (size 0.6) (drill 0.3) (layers "F.Cu" "B.Cu") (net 2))
 (via (at 134 121.8) (size 0.6) (drill 0.3) (layers "F.Cu" "B.Cu") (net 2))
 (via (at 138 121.8) (size 0.6) (drill 0.3) (layers "F.Cu" "B.Cu") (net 2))
 (via (at 142 121.8) (size 0.6) (drill 0.3) (layers "F.Cu" "B.Cu") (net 2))
 (via (at 146 121.8) (size 0.6) (drill 0.3) (layers "F.Cu" "B.Cu") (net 2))
 (via (at 106 125.8) (size 0.6) (drill 0.3) (layers "F.Cu" "B.Cu") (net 2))
 (via (at 110 125.8) (size 0.6) (drill 0.3) (layers "F.Cu" "B.Cu") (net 2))
 (via (at 114 125.8) (size 0.6) (drill 0.3) (layers "F.Cu" "B.Cu") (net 2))
 (via (at 118 125.8) (size 0.6) (drill 0.3) (layers "F.Cu" "B.Cu") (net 2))
 (via (at 122 125.8) (size 0.6) (drill 0.3) (layers "F.Cu" "B.Cu") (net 2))
 (via (at 134 125.8) (size 0.6) (drill 0.3) (layers "F.Cu" "B.Cu") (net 2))
 (via (at 138 125.8) (size 0.6) (drill 0.3) (layers "F.Cu" "B.Cu") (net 2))
 (via (at 142 125.8) (size 0.6) (drill 0.3) (layers "F.Cu" "B.Cu") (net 2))
 (via (at 146 125.8) (size 0.6) (drill 0.3) (layers "F.Cu" "B.Cu") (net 2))
 (via (at 106 129.8) (size 0.6) (drill 0.3) (layers "F.Cu" "B.Cu") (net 2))
 (via (at 110 129.8) (size 0.6) (drill 0.3) (layers "F.Cu" "B.Cu") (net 2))
 (via (at 114 129.8) (size 0.6) (drill 0.3) (layers "F.Cu" "B.Cu") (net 2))
 (via (at 118 129.8) (size 0.6) (drill 0.3) (layers "F.Cu" "B.Cu") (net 2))
 (via (at 122 129.8) (size 0.6) (drill 0.3) (layers "F.Cu" "B.Cu") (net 2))
 (via (at 134 129.8) (size 0.6) (drill 0.3) (layers "F.Cu" "B.Cu") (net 2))
 (via (at 138 129.8) (size 0.6) (drill 0.3) (layers "F.Cu" "B.Cu") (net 2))
 (via (at 142 129.8) (size 0.6) (drill 0.3) (layers "F.Cu" "B.Cu") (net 2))
 (via (at 146 129.8) (size 0.6) (drill 0.3) (layers "F.Cu" "B.Cu") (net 2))
 (via (at 106 133.8) (size 0.6) (drill 0.3) (layers "F.Cu" "B.Cu") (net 2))
 (via (at 110 133.8) (size 0.6) (drill 0.3) (layers "F.Cu" "B.Cu") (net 2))
 (via (at 114 133.8) (size 0.6) (drill 0.3) (layers "F.Cu" "B.Cu") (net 2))
 (via (at 118 133.8) (size 0.6) (drill 0.3) (layers "F.Cu" "B.Cu") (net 2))
 (via (at 122 133.8) (size 0.6) (drill 0.3) (layers "F.Cu" "B.Cu") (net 2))
 (via (at 134 133.8) (size 0.6) (drill 0.3) (layers "F.Cu" "B.Cu") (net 2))
 (via (at 138 133.8) (size 0.6) (drill 0.3) (layers "F.Cu" "B.Cu") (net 2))
 (via (at 142 133.8) (size 0.6) (drill 0.3) (layers "F.Cu" "B.Cu") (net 2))
 (via (at 146 133.8) (size 0.6) (drill 0.3) (layers "F.Cu" "B.Cu") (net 2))
 (via (at 106 137.8) (size 0.6) (drill 0.3) (layers "F.Cu" "B.Cu") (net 2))
 (via (at 110 137.8) (size 0.6) (drill 0.3) (layers "F.Cu" "B.Cu") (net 2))
 (via (at 114 137.8) (size 0.6) (drill 0.3) (layers "F.Cu" "B.Cu") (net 2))
 (via (at 118 137.8) (size 0.6) (drill 0.3) (layers "F.Cu" "B.Cu") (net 2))
 (via (at 122 137.8) (size 0.6) (drill 0.3) (layers "F.Cu" "B.Cu") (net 2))
 (via (at 134 137.8) (size 0.6) (drill 0.3) (layers "F.Cu" "B.Cu") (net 2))
 (via (at 138 137.8) (size 0.6) (drill 0.3) (layers "F.Cu" "B.Cu") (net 2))
 (via (at 142 137.8) (size 0.6) (drill 0.3) (layers "F.Cu" "B.Cu") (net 2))
 (via (at 146 137.8) (size 0.6) (drill 0.3) (layers "F.Cu" "B.Cu") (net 2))
 (via (at 106 141.8) (size 0.6) (drill 0.3) (layers "F.Cu" "B.Cu") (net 2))
 (via (at 110 141.8) (size 0.6) (drill 0.3) (layers "F.Cu" "B.Cu") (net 2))
 (via (at 114 141.8) (size 0.6) (drill 0.3) (layers "F.Cu" "B.Cu") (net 2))
 (via (at 118 141.8) (size 0.6) (drill 0.3) (layers "F.Cu" "B.Cu") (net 2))
 (via (at 122 141.8) (size 0.6) (drill 0.3) (layers "F.Cu" "B.Cu") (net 2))
 (via (at 134 141.8) (size 0.6) (drill 0.3) (layers "F.Cu" "B.Cu") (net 2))
 (via (at 138 141.8) (size 0.6) (drill 0.3) (layers "F.Cu" "B.Cu") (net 2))
 (via (at 142 141.8) (size 0.6) (drill 0.3) (layers "F.Cu" "B.Cu") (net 2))
 (via (at 146 141.8) (size 0.6) (drill 0.3) (layers "F.Cu" "B.Cu") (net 2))
 (via (at 106 145.8) (size 0.6) (drill 0.3) (layers "F.Cu" "B.Cu") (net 2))
 (via (at 110 145.8) (size 0.6) (drill 0.3) (layers "F.Cu" "B.Cu") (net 2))
 (via (at 114 145.8) (size 0.6) (drill 0.3) (layers "F.Cu" "B.Cu") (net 2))
 (via (at 118 145.8) (size 0.6) (drill 0.3) (layers "F.Cu" "B.Cu") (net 2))
 (via (at 122 145.8) (size 0.6) (drill 0.3) (layers "F.Cu" "B.Cu") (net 2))
 (via (at 134 145.8) (size 0.6) (drill 0.3) (layers "F.Cu" "B.Cu") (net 2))
 (via (at 138 145.8) (size 0.6) (drill 0.3) (layers "F.Cu" "B.Cu") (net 2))
 (via (at 142 145.8) (size 0.6) (drill 0.3) (layers "F.Cu" "B.Cu") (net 2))
 (via (at 146 145.8) (size 0.6) (drill 0.3) (layers "F.Cu" "B.Cu") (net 2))
 (via (at 131.9 99) (size 0.6) (drill 0.3) (layers "F.Cu" "B.Cu") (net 2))
 (via (at 131.9 92) (size 0.6) (drill 0.3) (layers "F.Cu" "B.Cu") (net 2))
 (via (at 125.3 143.525) (size 0.6) (drill 0.3) (layers "F.Cu" "B.Cu") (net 2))
 (via (at 129.7 143.525) (size 0.6) (drill 0.3) (layers "F.Cu" "B.Cu") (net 2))
 (via (at 125.3 146.475) (size 0.6) (drill 0.3) (layers "F.Cu" "B.Cu") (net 2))
 (via (at 129.7 146.475) (size 0.6) (drill 0.3) (layers "F.Cu" "B.Cu") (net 2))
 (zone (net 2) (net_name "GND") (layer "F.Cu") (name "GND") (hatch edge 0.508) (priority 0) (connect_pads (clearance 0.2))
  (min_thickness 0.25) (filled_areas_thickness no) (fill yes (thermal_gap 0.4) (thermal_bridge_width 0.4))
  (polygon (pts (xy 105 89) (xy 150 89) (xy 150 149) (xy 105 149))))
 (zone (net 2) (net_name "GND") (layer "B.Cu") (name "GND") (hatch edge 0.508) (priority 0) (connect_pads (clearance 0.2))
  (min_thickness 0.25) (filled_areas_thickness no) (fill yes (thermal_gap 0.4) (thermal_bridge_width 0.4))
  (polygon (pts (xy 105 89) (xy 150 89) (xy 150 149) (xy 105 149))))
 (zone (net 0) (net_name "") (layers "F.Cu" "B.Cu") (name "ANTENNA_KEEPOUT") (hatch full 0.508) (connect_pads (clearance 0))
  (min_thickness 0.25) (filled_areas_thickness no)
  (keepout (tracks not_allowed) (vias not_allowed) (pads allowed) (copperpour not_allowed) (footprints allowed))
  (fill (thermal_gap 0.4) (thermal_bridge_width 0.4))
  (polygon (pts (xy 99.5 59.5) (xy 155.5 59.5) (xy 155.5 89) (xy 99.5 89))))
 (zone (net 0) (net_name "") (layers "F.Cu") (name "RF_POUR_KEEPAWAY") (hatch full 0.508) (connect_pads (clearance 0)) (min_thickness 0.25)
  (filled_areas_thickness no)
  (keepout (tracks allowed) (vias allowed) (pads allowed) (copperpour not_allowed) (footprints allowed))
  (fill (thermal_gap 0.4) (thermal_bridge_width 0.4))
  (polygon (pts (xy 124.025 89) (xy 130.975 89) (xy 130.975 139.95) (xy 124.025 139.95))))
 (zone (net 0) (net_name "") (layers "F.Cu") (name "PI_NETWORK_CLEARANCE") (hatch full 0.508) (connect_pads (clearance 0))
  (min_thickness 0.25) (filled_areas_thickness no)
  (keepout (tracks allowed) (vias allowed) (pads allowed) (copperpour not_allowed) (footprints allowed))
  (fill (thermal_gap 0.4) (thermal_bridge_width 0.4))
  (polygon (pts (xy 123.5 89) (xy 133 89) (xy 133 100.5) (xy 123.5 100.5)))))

